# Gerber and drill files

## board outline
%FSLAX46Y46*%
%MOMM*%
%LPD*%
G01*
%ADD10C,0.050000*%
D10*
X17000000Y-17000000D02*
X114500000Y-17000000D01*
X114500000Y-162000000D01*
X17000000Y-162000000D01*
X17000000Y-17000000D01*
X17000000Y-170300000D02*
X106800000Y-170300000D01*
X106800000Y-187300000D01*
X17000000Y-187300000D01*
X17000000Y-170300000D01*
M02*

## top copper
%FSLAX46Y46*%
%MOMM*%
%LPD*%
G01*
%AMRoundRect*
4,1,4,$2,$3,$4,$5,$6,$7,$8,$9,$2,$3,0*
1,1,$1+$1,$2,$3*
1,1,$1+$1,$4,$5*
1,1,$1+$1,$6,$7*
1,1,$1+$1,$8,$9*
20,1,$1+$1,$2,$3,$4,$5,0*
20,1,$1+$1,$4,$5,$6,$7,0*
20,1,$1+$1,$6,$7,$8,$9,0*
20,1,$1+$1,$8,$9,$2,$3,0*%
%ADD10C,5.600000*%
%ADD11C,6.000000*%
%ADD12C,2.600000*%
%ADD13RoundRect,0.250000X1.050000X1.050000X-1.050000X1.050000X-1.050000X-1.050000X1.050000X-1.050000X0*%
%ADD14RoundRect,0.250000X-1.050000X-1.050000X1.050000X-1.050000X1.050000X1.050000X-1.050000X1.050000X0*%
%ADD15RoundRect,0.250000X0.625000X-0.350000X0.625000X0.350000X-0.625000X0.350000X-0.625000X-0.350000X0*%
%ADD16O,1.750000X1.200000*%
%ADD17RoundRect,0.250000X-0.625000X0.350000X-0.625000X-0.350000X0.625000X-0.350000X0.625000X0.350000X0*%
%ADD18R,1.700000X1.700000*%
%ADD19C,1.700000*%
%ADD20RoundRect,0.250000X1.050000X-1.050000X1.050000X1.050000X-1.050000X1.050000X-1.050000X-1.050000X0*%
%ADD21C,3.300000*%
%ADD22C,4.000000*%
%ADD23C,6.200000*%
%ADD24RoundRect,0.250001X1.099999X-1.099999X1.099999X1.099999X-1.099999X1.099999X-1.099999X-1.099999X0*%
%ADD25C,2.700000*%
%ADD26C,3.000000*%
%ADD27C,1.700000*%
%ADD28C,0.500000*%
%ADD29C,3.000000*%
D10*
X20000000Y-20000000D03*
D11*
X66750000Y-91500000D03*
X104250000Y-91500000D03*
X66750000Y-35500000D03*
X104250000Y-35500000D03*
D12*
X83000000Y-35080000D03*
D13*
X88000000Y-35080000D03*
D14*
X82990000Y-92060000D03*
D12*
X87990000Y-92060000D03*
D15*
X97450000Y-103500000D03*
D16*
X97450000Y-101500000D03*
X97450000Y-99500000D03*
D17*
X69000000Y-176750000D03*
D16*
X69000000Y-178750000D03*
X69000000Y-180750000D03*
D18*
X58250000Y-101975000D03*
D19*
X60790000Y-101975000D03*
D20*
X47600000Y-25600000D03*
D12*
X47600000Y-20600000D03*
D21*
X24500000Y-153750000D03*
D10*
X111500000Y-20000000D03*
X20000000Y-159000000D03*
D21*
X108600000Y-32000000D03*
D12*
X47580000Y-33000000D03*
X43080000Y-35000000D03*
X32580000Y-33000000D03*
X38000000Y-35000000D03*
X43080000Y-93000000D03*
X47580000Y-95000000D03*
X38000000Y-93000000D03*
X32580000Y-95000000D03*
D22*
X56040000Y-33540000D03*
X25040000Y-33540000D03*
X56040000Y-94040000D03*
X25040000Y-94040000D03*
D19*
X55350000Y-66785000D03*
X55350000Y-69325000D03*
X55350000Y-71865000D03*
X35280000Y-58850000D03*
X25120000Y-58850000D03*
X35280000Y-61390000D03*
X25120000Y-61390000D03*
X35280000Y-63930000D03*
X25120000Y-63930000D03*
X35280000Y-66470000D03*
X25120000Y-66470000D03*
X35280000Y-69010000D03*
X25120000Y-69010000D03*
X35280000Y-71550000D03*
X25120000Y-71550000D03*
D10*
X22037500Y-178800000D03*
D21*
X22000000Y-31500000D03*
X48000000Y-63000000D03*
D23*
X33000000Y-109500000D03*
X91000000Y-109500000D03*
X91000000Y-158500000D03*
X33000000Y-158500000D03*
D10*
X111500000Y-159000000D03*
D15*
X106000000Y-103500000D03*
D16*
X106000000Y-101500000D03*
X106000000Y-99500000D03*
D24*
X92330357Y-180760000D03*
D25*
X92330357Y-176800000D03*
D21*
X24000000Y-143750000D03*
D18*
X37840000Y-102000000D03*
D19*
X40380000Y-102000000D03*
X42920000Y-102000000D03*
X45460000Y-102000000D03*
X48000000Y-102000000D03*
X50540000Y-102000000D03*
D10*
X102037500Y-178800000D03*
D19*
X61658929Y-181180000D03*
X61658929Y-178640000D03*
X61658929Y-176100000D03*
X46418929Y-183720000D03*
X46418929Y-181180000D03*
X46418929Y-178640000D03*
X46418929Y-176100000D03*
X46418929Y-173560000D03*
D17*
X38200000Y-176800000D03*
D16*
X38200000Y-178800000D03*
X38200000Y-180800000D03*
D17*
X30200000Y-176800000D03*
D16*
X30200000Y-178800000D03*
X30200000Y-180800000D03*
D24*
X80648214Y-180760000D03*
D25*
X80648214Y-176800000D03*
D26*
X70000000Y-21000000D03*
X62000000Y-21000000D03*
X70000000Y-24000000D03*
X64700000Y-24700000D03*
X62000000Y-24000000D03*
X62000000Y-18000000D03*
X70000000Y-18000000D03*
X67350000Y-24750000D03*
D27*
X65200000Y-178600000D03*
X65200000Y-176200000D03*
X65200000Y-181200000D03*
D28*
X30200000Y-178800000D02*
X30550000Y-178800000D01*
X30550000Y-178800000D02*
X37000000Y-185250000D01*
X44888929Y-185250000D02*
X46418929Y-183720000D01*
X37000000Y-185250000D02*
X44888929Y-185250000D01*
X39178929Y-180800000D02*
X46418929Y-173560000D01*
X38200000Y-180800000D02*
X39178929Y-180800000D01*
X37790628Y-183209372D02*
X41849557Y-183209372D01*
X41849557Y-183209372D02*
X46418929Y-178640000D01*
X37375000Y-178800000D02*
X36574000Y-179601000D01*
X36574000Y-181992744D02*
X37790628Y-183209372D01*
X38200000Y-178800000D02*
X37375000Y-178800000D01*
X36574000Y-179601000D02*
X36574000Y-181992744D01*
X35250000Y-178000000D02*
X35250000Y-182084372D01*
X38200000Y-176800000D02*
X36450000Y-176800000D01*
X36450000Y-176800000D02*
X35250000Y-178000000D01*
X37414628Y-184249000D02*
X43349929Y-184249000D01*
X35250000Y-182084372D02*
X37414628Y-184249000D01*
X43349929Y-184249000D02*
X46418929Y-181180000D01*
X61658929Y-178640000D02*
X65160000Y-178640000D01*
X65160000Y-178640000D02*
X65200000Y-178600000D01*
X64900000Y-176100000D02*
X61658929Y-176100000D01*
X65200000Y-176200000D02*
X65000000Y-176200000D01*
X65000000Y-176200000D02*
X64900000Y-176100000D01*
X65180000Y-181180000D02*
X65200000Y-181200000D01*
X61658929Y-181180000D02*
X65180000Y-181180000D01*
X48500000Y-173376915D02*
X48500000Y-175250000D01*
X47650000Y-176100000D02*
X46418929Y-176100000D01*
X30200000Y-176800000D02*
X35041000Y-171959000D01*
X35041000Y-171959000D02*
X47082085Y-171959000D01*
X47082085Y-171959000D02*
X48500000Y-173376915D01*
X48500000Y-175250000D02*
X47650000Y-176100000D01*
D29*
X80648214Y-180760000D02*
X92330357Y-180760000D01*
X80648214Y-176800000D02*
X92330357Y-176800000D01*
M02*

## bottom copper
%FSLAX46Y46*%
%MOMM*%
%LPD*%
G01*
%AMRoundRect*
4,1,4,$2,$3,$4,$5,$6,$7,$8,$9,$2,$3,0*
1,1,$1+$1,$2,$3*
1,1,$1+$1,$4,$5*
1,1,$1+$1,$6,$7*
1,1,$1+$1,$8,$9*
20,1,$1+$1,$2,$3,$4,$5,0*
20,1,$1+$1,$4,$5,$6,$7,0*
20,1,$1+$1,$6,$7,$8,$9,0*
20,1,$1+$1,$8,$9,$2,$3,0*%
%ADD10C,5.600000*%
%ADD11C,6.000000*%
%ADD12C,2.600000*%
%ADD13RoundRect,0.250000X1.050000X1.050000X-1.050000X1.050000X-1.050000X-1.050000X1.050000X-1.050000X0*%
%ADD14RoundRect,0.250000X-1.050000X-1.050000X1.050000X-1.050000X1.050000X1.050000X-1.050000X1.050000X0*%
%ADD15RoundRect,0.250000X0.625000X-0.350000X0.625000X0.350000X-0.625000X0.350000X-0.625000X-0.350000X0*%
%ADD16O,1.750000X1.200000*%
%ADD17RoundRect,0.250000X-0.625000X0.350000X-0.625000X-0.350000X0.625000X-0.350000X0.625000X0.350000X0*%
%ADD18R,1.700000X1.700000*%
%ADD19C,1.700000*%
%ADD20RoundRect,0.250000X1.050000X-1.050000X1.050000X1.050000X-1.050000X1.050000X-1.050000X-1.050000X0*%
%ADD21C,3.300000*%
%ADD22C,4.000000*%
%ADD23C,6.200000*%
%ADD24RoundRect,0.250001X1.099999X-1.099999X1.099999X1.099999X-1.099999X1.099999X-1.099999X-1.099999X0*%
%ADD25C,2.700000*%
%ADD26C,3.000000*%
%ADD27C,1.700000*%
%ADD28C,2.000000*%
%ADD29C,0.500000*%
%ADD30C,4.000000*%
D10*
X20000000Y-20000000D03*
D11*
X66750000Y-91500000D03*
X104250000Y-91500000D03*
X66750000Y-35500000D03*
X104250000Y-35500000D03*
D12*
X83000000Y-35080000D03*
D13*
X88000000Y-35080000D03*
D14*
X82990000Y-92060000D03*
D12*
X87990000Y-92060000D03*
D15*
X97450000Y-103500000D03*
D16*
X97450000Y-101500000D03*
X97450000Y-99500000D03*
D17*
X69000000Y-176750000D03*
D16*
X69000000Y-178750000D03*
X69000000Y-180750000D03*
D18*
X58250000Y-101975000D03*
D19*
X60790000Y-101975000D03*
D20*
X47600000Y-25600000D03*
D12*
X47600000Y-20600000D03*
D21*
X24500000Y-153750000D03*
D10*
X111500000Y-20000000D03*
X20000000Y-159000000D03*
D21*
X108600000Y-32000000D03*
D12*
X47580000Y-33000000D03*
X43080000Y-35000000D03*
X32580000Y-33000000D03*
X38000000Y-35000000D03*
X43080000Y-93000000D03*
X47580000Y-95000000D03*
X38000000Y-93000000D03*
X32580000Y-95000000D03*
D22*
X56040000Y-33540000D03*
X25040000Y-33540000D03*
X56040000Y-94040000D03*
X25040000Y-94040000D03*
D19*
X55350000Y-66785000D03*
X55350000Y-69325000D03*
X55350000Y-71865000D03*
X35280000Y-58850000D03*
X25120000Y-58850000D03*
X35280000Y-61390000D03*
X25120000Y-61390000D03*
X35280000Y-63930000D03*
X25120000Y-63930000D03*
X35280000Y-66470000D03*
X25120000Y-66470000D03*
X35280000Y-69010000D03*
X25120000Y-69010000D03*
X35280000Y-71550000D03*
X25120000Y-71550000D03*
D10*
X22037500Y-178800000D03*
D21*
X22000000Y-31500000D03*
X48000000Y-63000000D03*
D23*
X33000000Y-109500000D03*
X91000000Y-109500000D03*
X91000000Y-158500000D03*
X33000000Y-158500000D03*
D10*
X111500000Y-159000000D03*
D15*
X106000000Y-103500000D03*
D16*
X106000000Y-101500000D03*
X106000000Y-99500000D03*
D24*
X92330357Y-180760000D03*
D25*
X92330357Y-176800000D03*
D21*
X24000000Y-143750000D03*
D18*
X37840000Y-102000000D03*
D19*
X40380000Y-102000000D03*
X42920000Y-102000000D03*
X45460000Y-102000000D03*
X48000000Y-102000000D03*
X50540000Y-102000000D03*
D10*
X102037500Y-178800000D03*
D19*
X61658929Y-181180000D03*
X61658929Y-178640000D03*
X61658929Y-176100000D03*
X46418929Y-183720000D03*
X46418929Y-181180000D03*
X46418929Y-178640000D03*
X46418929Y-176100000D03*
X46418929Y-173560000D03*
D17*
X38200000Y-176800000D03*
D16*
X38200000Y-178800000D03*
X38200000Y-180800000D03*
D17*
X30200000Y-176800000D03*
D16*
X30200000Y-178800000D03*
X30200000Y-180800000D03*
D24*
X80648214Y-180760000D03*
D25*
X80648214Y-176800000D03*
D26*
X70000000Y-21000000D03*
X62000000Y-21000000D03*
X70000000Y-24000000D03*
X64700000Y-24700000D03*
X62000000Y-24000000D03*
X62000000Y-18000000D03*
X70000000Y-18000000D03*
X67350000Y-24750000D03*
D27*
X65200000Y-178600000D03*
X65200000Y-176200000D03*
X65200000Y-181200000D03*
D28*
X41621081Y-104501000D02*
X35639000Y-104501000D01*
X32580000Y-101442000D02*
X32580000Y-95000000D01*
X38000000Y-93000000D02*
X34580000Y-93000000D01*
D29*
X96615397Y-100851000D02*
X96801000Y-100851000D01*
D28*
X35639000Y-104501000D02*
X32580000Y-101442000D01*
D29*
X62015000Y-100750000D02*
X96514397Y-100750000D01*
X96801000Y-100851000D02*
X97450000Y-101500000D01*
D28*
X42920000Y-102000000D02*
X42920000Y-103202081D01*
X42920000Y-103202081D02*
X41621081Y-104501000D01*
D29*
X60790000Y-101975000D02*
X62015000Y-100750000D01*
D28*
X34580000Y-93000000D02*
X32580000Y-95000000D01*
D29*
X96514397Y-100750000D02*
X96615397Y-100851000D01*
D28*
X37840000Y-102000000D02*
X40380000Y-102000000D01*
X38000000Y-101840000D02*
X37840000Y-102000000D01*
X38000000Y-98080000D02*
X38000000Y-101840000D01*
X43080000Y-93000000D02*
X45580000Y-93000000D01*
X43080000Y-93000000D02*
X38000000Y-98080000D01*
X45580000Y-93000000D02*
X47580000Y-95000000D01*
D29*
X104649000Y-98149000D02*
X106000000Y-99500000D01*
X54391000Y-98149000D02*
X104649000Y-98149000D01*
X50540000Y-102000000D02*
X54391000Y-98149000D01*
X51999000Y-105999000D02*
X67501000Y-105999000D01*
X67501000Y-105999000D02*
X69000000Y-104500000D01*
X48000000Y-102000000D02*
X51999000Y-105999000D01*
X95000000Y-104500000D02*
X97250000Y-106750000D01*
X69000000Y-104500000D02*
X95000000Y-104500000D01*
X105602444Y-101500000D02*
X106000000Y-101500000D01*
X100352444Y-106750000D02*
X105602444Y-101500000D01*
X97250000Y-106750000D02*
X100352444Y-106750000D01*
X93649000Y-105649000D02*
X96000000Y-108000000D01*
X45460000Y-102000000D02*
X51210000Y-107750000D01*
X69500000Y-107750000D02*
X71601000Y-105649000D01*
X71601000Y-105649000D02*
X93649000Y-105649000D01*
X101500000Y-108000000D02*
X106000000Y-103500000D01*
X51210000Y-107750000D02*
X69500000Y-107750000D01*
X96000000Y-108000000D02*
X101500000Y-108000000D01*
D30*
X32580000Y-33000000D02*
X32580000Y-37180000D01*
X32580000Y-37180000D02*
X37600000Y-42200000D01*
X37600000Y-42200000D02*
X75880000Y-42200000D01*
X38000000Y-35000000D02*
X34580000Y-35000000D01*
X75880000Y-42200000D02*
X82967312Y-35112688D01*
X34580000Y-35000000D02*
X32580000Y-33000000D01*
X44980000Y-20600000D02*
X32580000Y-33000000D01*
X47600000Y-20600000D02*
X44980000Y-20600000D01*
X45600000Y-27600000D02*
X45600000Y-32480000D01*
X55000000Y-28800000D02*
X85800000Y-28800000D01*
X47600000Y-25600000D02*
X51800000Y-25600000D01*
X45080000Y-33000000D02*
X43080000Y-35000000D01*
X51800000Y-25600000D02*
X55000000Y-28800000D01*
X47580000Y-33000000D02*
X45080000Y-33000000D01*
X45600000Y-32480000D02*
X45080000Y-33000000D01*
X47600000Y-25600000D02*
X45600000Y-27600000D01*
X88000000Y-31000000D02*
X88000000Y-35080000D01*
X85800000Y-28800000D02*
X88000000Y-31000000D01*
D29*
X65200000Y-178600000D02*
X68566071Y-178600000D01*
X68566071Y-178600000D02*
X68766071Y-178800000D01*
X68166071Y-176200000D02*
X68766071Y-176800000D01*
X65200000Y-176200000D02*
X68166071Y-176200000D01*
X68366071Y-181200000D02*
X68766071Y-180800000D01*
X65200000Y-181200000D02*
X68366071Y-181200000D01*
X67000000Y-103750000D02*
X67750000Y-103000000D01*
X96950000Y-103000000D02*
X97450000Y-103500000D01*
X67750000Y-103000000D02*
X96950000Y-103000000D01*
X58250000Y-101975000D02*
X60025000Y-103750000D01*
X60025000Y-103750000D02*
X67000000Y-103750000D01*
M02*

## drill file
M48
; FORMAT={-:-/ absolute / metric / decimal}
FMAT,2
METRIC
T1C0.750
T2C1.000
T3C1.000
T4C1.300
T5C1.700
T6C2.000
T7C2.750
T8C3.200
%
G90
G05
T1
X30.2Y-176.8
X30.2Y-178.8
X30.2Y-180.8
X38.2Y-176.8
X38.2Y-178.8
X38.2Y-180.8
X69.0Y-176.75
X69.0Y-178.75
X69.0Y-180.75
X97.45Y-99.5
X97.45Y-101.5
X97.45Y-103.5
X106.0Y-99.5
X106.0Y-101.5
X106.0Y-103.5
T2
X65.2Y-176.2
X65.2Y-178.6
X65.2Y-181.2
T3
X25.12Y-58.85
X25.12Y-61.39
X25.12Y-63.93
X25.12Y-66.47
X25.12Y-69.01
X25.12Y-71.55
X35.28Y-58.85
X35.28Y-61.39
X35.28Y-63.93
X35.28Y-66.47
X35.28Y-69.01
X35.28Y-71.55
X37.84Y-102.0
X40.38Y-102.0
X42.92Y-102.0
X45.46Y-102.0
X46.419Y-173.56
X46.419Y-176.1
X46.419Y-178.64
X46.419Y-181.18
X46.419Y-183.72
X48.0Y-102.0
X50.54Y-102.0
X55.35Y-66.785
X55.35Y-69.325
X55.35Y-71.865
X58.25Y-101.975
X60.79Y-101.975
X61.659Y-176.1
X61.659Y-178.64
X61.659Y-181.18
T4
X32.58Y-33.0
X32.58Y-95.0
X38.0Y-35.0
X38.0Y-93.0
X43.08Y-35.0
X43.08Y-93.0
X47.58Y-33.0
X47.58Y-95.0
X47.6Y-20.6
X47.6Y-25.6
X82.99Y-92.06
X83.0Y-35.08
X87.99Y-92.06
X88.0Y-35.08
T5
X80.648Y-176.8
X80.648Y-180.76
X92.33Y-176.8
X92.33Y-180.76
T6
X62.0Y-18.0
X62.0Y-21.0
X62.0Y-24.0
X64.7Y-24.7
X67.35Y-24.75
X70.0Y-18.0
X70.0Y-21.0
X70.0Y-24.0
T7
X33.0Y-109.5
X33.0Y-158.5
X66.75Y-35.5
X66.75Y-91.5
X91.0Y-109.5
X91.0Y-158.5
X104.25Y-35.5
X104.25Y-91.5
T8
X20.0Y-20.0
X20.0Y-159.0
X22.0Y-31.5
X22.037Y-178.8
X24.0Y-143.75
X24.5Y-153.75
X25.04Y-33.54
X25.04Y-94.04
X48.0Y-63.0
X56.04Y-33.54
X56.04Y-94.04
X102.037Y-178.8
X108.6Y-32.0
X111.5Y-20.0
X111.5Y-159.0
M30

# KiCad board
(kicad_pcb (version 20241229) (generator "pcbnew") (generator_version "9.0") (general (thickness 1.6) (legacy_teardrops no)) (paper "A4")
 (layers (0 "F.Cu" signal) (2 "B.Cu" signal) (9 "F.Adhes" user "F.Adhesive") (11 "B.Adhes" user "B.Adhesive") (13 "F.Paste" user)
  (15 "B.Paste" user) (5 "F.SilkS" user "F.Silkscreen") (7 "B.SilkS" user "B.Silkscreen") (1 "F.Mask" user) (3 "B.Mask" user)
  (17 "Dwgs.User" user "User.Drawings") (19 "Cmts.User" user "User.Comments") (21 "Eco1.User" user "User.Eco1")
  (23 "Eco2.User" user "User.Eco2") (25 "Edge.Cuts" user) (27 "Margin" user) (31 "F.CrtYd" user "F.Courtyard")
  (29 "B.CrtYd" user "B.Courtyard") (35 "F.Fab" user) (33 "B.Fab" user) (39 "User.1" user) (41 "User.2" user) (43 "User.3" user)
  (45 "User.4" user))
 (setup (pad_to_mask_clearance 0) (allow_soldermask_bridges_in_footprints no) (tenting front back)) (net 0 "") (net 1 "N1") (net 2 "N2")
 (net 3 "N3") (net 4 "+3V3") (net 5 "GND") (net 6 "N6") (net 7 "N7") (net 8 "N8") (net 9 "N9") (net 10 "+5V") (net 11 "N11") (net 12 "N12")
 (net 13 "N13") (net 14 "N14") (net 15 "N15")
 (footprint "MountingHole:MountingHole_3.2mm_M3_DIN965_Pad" (layer "F.Cu") (at 20 20)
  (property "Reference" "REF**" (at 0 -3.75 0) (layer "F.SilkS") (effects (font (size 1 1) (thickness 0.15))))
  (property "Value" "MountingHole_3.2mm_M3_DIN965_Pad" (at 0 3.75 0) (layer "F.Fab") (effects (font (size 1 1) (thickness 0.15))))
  (pad "1" thru_hole circle (at 0 0) (size 5.6 5.6) (drill 3.2) (layers "*.Cu" "*.Mask") (remove_unused_layers no) (zone_connect 2)))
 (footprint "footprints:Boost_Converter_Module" (layer "F.Cu") (at 85.5 63.5 90)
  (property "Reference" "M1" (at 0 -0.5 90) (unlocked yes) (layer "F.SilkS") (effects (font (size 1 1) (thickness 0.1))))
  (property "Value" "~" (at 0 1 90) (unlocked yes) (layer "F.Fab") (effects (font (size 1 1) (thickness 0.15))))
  (pad "" thru_hole circle (at -28 -18.75 90) (size 6 6) (drill 2.75) (layers "*.Cu" "*.Mask") (remove_unused_layers no))
  (pad "" thru_hole circle (at -28 18.75 90) (size 6 6) (drill 2.75) (layers "*.Cu" "*.Mask") (remove_unused_layers no))
  (pad "" thru_hole circle (at 28 -18.75 90) (size 6 6) (drill 2.75) (layers "*.Cu" "*.Mask") (remove_unused_layers no))
  (pad "" thru_hole circle (at 28 18.75 90) (size 6 6) (drill 2.75) (layers "*.Cu" "*.Mask") (remove_unused_layers no))
  (pad "1" thru_hole circle (at 28.42 -2.5 180) (size 2.6 2.6) (drill 1.3) (layers "*.Cu" "*.Mask") (remove_unused_layers no) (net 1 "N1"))
  (pad "2" thru_hole roundrect (at 28.42 2.5 180) (size 2.6 2.6) (drill 1.3) (layers "*.Cu" "*.Mask") (remove_unused_layers no)
   (roundrect_rratio 0.096154) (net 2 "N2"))
  (pad "3" thru_hole roundrect (at -28.56 -2.51) (size 2.6 2.6) (drill 1.3) (layers "*.Cu" "*.Mask") (remove_unused_layers no)
   (roundrect_rratio 0.096154) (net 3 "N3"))
  (pad "4" thru_hole circle (at -28.56 2.49) (size 2.6 2.6) (drill 1.3) (layers "*.Cu" "*.Mask") (remove_unused_layers no)))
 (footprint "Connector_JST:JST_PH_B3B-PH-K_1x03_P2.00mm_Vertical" (layer "F.Cu") (at 97.45 103.5 90)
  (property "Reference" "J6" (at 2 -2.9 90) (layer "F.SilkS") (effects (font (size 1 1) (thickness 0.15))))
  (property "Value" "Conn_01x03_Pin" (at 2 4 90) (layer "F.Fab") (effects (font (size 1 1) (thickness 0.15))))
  (pad "1" thru_hole roundrect (at 0 0 90) (size 1.2 1.75) (drill 0.75) (layers "*.Cu" "*.Mask") (remove_unused_layers no)
   (roundrect_rratio 0.208333) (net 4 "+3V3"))
  (pad "2" thru_hole oval (at 2 0 90) (size 1.2 1.75) (drill 0.75) (layers "*.Cu" "*.Mask") (remove_unused_layers no) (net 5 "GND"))
  (pad "3" thru_hole oval (at 4 0 90) (size 1.2 1.75) (drill 0.75) (layers "*.Cu" "*.Mask") (remove_unused_layers no) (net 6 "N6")))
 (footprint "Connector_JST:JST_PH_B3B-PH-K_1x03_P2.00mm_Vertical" (layer "F.Cu") (at 69 176.75 -90)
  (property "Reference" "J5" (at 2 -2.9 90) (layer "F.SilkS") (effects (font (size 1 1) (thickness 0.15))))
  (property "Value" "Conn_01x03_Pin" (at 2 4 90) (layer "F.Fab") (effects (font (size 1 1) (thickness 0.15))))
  (pad "1" thru_hole roundrect (at 0 0 270) (size 1.2 1.75) (drill 0.75) (layers "*.Cu" "*.Mask") (remove_unused_layers no)
   (roundrect_rratio 0.208333) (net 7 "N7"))
  (pad "2" thru_hole oval (at 2 0 270) (size 1.2 1.75) (drill 0.75) (layers "*.Cu" "*.Mask") (remove_unused_layers no) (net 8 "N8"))
  (pad "3" thru_hole oval (at 4 0 270) (size 1.2 1.75) (drill 0.75) (layers "*.Cu" "*.Mask") (remove_unused_layers no) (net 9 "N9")))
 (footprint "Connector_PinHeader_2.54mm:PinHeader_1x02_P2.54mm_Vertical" (layer "F.Cu") (at 58.25 101.975 90)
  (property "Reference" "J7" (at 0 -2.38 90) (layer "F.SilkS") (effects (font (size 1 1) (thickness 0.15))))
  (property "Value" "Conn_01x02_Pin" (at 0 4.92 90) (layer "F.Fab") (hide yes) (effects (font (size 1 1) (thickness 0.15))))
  (pad "1" thru_hole rect (at 0 0 90) (size 1.7 1.7) (drill 1) (layers "*.Cu" "*.Mask") (remove_unused_layers no) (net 4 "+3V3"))
  (pad "2" thru_hole circle (at 0 2.54 90) (size 1.7 1.7) (drill 1) (layers "*.Cu" "*.Mask") (remove_unused_layers no) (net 5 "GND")))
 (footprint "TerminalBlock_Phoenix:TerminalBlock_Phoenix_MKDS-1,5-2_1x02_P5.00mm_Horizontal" (layer "F.Cu") (at 47.6 25.6 90)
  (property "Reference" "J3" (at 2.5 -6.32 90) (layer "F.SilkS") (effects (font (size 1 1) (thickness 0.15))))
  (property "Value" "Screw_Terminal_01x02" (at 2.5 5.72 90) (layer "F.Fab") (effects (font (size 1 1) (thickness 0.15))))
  (pad "1" thru_hole roundrect (at 0 0 90) (size 2.6 2.6) (drill 1.3) (layers "*.Cu" "*.Mask") (remove_unused_layers no)
   (roundrect_rratio 0.096154) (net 2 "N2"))
  (pad "2" thru_hole circle (at 5 0 90) (size 2.6 2.6) (drill 1.3) (layers "*.Cu" "*.Mask") (remove_unused_layers no) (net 1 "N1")))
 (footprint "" (layer "F.Cu") (at 24.5 153.75)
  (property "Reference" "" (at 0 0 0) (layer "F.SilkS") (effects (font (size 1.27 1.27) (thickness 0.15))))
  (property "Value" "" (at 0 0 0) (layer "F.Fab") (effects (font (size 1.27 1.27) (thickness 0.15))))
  (pad "1" thru_hole circle (at 0 0) (size 3.3 3.3) (drill 3.2) (layers "*.Cu" "*.Mask") (remove_unused_layers no) (zone_connect 2)))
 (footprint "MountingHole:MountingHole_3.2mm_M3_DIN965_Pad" (layer "F.Cu") (at 111.5 20)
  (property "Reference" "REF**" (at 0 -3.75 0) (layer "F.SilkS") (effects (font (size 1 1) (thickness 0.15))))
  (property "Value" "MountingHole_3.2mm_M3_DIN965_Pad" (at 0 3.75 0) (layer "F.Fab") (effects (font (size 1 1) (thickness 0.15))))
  (pad "1" thru_hole circle (at 0 0) (size 5.6 5.6) (drill 3.2) (layers "*.Cu" "*.Mask") (remove_unused_layers no) (zone_connect 2)))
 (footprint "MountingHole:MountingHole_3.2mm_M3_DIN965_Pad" (layer "F.Cu") (at 20 159)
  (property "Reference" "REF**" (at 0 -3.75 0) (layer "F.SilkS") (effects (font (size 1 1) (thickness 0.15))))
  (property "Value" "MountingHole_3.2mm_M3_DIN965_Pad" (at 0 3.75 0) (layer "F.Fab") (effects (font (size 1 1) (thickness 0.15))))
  (pad "1" thru_hole circle (at 0 0) (size 5.6 5.6) (drill 3.2) (layers "*.Cu" "*.Mask") (remove_unused_layers no) (zone_connect 2)))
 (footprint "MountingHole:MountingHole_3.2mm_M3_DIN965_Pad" (layer "F.Cu") (at 108.6 32)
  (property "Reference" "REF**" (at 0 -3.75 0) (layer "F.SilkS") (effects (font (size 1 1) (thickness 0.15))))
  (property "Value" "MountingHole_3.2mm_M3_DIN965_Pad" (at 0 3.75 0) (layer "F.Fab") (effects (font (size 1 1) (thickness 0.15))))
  (pad "1" thru_hole circle (at 0 0) (size 3.3 3.3) (drill 3.2) (layers "*.Cu" "*.Mask") (remove_unused_layers no) (zone_connect 2)))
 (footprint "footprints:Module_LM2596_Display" (layer "F.Cu") (at 58.58 64 -90)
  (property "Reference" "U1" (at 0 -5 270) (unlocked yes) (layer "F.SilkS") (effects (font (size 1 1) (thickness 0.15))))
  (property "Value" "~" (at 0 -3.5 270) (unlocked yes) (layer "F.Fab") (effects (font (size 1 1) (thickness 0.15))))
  (pad "1" thru_hole circle (at -31 11 270) (size 2.6 2.6) (drill 1.3) (layers "*.Cu" "*.Mask") (remove_unused_layers no) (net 2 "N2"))
  (pad "1" thru_hole circle (at -29 15.5 270) (size 2.6 2.6) (drill 1.3) (layers "*.Cu" "*.Mask") (remove_unused_layers no) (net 2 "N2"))
  (pad "2" thru_hole circle (at -31 26 270) (size 2.6 2.6) (drill 1.3) (layers "*.Cu" "*.Mask") (remove_unused_layers no) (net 1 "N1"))
  (pad "2" thru_hole circle (at -29 20.58 270) (size 2.6 2.6) (drill 1.3) (layers "*.Cu" "*.Mask") (remove_unused_layers no) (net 1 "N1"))
  (pad "3" thru_hole circle (at 29 15.5 270) (size 2.6 2.6) (drill 1.3) (layers "*.Cu" "*.Mask") (remove_unused_layers no) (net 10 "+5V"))
  (pad "3" thru_hole circle (at 31 11 270) (size 2.6 2.6) (drill 1.3) (layers "*.Cu" "*.Mask") (remove_unused_layers no) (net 10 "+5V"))
  (pad "4" thru_hole circle (at 29 20.58 270) (size 2.6 2.6) (drill 1.3) (layers "*.Cu" "*.Mask") (remove_unused_layers no) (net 5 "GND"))
  (pad "4" thru_hole circle (at 31 26 270) (size 2.6 2.6) (drill 1.3) (layers "*.Cu" "*.Mask") (remove_unused_layers no) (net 5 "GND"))
  (pad "5" thru_hole circle (at -30.46 2.54 270) (size 4 4) (drill 3.2) (layers "*.Cu" "*.Mask") (remove_unused_layers no))
  (pad "5" thru_hole circle (at -30.46 33.54 270) (size 4 4) (drill 3.2) (layers "*.Cu" "*.Mask") (remove_unused_layers no))
  (pad "5" thru_hole circle (at 30.04 2.54 270) (size 4 4) (drill 3.2) (layers "*.Cu" "*.Mask") (remove_unused_layers no))
  (pad "5" thru_hole circle (at 30.04 33.54 270) (size 4 4) (drill 3.2) (layers "*.Cu" "*.Mask") (remove_unused_layers no))
  (pad "6" thru_hole circle (at 2.785 3.23 90) (size 1.7 1.7) (drill 1) (layers "*.Cu" "*.Mask") (remove_unused_layers no))
  (pad "7" thru_hole circle (at 5.325 3.23 90) (size 1.7 1.7) (drill 1) (layers "*.Cu" "*.Mask") (remove_unused_layers no))
  (pad "8" thru_hole circle (at 7.865 3.23 90) (size 1.7 1.7) (drill 1) (layers "*.Cu" "*.Mask") (remove_unused_layers no))
  (pad "9" thru_hole circle (at -5.15 23.3 270) (size 1.7 1.7) (drill 1) (layers "*.Cu" "*.Mask") (remove_unused_layers no))
  (pad "9" thru_hole circle (at -5.15 33.46 270) (size 1.7 1.7) (drill 1) (layers "*.Cu" "*.Mask") (remove_unused_layers no))
  (pad "9" thru_hole circle (at -2.61 23.3 270) (size 1.7 1.7) (drill 1) (layers "*.Cu" "*.Mask") (remove_unused_layers no))
  (pad "9" thru_hole circle (at -2.61 33.46 270) (size 1.7 1.7) (drill 1) (layers "*.Cu" "*.Mask") (remove_unused_layers no))
  (pad "9" thru_hole circle (at -0.07 23.3 270) (size 1.7 1.7) (drill 1) (layers "*.Cu" "*.Mask") (remove_unused_layers no))
  (pad "9" thru_hole circle (at -0.07 33.46 270) (size 1.7 1.7) (drill 1) (layers "*.Cu" "*.Mask") (remove_unused_layers no))
  (pad "9" thru_hole circle (at 2.47 23.3 270) (size 1.7 1.7) (drill 1) (layers "*.Cu" "*.Mask" "Eco1.User") (remove_unused_layers no))
  (pad "9" thru_hole circle (at 2.47 33.46 270) (size 1.7 1.7) (drill 1) (layers "*.Cu" "*.Mask") (remove_unused_layers no))
  (pad "9" thru_hole circle (at 5.01 23.3 270) (size 1.7 1.7) (drill 1) (layers "*.Cu" "*.Mask") (remove_unused_layers no))
  (pad "9" thru_hole circle (at 5.01 33.46 270) (size 1.7 1.7) (drill 1) (layers "*.Cu" "*.Mask") (remove_unused_layers no))
  (pad "9" thru_hole circle (at 7.55 23.3 270) (size 1.7 1.7) (drill 1) (layers "*.Cu" "*.Mask") (remove_unused_layers no))
  (pad "9" thru_hole circle (at 7.55 33.46 270) (size 1.7 1.7) (drill 1) (layers "*.Cu" "*.Mask") (remove_unused_layers no)))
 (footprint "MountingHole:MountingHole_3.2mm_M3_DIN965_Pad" (layer "F.Cu") (at 22.0375 178.8)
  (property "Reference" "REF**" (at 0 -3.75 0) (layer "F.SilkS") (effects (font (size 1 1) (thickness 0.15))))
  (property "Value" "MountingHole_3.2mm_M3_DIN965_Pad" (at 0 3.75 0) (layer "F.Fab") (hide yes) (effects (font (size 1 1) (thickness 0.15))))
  (pad "1" thru_hole circle (at 0 0) (size 5.6 5.6) (drill 3.2) (layers "*.Cu" "*.Mask") (remove_unused_layers no) (zone_connect 2)))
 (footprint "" (layer "F.Cu") (at 22 31.5)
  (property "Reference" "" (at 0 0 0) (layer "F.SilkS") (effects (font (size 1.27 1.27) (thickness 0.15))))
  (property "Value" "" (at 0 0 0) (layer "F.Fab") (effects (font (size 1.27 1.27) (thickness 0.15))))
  (pad "1" thru_hole circle (at 0 0) (size 3.3 3.3) (drill 3.2) (layers "*.Cu" "*.Mask") (remove_unused_layers no) (zone_connect 2)))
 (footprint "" (layer "F.Cu") (at 48 63)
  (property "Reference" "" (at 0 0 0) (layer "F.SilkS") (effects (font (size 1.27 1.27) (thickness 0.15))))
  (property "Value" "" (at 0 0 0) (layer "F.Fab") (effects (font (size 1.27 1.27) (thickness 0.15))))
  (pad "1" thru_hole circle (at 0 0) (size 3.3 3.3) (drill 3.2) (layers "*.Cu" "*.Mask") (remove_unused_layers no) (zone_connect 2)))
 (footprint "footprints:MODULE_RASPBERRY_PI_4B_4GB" (layer "F.Cu") (at 72 134)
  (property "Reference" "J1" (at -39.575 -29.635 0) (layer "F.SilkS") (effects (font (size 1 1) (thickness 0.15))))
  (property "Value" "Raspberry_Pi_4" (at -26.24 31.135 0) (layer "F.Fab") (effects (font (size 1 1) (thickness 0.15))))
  (pad "S1" thru_hole circle (at -39 -24.5) (size 6.2 6.2) (drill 2.75) (layers "*.Cu" "*.Mask") (remove_unused_layers no)
   (solder_mask_margin 0.102))
  (pad "S2" thru_hole circle (at 19 -24.5) (size 6.2 6.2) (drill 2.75) (layers "*.Cu" "*.Mask") (remove_unused_layers no)
   (solder_mask_margin 0.102))
  (pad "S3" thru_hole circle (at 19 24.5) (size 6.2 6.2) (drill 2.75) (layers "*.Cu" "*.Mask") (remove_unused_layers no)
   (solder_mask_margin 0.102))
  (pad "S4" thru_hole circle (at -39 24.5) (size 6.2 6.2) (drill 2.75) (layers "*.Cu" "*.Mask") (remove_unused_layers no)
   (solder_mask_margin 0.102)))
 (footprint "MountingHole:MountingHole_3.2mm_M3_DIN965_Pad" (layer "F.Cu") (at 111.5 159)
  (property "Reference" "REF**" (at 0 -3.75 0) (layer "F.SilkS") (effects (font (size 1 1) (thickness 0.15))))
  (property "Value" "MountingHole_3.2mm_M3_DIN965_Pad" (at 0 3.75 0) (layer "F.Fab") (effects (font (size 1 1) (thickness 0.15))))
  (pad "1" thru_hole circle (at 0 0) (size 5.6 5.6) (drill 3.2) (layers "*.Cu" "*.Mask") (remove_unused_layers no) (zone_connect 2)))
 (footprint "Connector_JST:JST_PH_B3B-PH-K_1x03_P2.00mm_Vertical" (layer "F.Cu") (at 106 103.5 90)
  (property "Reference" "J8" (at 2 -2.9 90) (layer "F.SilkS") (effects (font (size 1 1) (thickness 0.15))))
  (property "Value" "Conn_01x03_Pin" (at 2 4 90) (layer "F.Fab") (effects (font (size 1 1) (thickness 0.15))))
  (pad "1" thru_hole roundrect (at 0 0 90) (size 1.2 1.75) (drill 0.75) (layers "*.Cu" "*.Mask") (remove_unused_layers no)
   (roundrect_rratio 0.208333) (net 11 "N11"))
  (pad "2" thru_hole oval (at 2 0 90) (size 1.2 1.75) (drill 0.75) (layers "*.Cu" "*.Mask") (remove_unused_layers no) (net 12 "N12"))
  (pad "3" thru_hole oval (at 4 0 90) (size 1.2 1.75) (drill 0.75) (layers "*.Cu" "*.Mask") (remove_unused_layers no) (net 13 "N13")))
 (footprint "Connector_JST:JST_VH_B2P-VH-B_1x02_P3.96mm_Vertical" (layer "F.Cu") (at 92.330357 180.76 90)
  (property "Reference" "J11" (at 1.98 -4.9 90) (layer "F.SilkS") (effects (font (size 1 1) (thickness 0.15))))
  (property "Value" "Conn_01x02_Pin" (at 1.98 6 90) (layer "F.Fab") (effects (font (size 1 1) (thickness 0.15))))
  (pad "1" thru_hole roundrect (at 0 0 90) (size 2.7 2.7) (drill 1.7) (layers "*.Cu" "*.Mask") (remove_unused_layers no)
   (roundrect_rratio 0.092593) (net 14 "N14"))
  (pad "2" thru_hole circle (at 3.96 0 90) (size 2.7 2.7) (drill 1.7) (layers "*.Cu" "*.Mask") (remove_unused_layers no) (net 3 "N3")))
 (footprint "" (layer "F.Cu") (at 24 143.75)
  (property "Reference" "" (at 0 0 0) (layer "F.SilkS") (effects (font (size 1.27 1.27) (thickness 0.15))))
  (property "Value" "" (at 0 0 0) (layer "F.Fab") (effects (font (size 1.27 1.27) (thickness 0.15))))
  (pad "1" thru_hole circle (at 0 0) (size 3.3 3.3) (drill 3.2) (layers "*.Cu" "*.Mask") (remove_unused_layers no) (zone_connect 2)))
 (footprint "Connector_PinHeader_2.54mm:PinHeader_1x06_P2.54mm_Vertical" (layer "F.Cu") (at 37.84 102 90)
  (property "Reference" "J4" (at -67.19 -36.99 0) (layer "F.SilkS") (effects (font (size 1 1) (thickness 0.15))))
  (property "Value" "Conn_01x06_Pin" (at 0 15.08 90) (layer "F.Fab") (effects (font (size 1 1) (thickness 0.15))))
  (pad "1" thru_hole rect (at 0 0 90) (size 1.7 1.7) (drill 1) (layers "*.Cu" "*.Mask") (remove_unused_layers no) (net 10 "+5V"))
  (pad "2" thru_hole circle (at 0 2.54 90) (size 1.7 1.7) (drill 1) (layers "*.Cu" "*.Mask") (remove_unused_layers no) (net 10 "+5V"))
  (pad "3" thru_hole circle (at 0 5.08 90) (size 1.7 1.7) (drill 1) (layers "*.Cu" "*.Mask") (remove_unused_layers no) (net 5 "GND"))
  (pad "4" thru_hole circle (at 0 7.62 90) (size 1.7 1.7) (drill 1) (layers "*.Cu" "*.Mask") (remove_unused_layers no) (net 11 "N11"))
  (pad "5" thru_hole circle (at 0 10.16 90) (size 1.7 1.7) (drill 1) (layers "*.Cu" "*.Mask") (remove_unused_layers no) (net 12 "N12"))
  (pad "6" thru_hole circle (at 0 12.7 90) (size 1.7 1.7) (drill 1) (layers "*.Cu" "*.Mask") (remove_unused_layers no) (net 13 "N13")))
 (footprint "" (layer "F.Cu") (at 102.0375 178.8)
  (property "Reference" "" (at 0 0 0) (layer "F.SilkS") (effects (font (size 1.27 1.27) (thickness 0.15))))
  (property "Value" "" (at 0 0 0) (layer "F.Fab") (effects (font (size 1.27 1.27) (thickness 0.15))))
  (pad "1" thru_hole circle (at 0 0) (size 5.6 5.6) (drill 3.2) (layers "*.Cu" "*.Mask") (remove_unused_layers no) (zone_connect 2)))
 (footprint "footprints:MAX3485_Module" (layer "B.Cu") (at 57.658929 174.14 90)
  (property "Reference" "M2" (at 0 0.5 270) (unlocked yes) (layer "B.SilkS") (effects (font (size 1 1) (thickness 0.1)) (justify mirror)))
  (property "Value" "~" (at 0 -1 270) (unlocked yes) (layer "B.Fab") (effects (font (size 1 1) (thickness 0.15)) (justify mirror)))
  (pad "1" thru_hole circle (at -7.04 4 90) (size 1.7 1.7) (drill 1) (layers "*.Cu" "*.Mask") (remove_unused_layers no) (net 7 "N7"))
  (pad "2" thru_hole circle (at -4.5 4 90) (size 1.7 1.7) (drill 1) (layers "*.Cu" "*.Mask") (remove_unused_layers no) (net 8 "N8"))
  (pad "3" thru_hole circle (at -1.96 4 90) (size 1.7 1.7) (drill 1) (layers "*.Cu" "*.Mask") (remove_unused_layers no) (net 9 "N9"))
  (pad "4" thru_hole circle (at -9.58 -11.24 90) (size 1.7 1.7) (drill 1) (layers "*.Cu" "*.Mask") (remove_unused_layers no) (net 5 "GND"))
  (pad "5" thru_hole circle (at -7.04 -11.24 90) (size 1.7 1.7) (drill 1) (layers "*.Cu" "*.Mask") (remove_unused_layers no) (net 11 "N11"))
  (pad "6" thru_hole circle (at -4.5 -11.24 90) (size 1.7 1.7) (drill 1) (layers "*.Cu" "*.Mask") (remove_unused_layers no) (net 12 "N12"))
  (pad "7" thru_hole circle (at -1.96 -11.24 90) (size 1.7 1.7) (drill 1) (layers "*.Cu" "*.Mask") (remove_unused_layers no) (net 4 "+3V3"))
  (pad "8" thru_hole circle (at 0.58 -11.24 90) (size 1.7 1.7) (drill 1) (layers "*.Cu" "*.Mask") (remove_unused_layers no) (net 13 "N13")))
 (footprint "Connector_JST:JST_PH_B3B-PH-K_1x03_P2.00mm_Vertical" (layer "B.Cu") (at 38.2 176.8 -90)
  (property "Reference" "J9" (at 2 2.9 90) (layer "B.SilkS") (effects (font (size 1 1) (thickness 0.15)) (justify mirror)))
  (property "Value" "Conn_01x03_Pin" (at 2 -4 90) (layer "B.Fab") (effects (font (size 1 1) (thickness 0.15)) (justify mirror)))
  (pad "1" thru_hole roundrect (at 0 0 270) (size 1.2 1.75) (drill 0.75) (layers "*.Cu" "*.Mask") (remove_unused_layers no)
   (roundrect_rratio 0.208333) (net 11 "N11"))
  (pad "2" thru_hole oval (at 2 0 270) (size 1.2 1.75) (drill 0.75) (layers "*.Cu" "*.Mask") (remove_unused_layers no) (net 12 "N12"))
  (pad "3" thru_hole oval (at 4 0 270) (size 1.2 1.75) (drill 0.75) (layers "*.Cu" "*.Mask") (remove_unused_layers no) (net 13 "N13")))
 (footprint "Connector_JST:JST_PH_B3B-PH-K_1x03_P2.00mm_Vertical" (layer "B.Cu") (at 30.2 176.8 -90)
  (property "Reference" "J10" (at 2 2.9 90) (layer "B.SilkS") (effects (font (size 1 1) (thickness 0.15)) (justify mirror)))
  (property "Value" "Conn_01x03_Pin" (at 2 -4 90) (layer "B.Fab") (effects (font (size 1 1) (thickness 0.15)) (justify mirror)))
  (pad "1" thru_hole roundrect (at 0 0 270) (size 1.2 1.75) (drill 0.75) (layers "*.Cu" "*.Mask") (remove_unused_layers no)
   (roundrect_rratio 0.208333) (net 4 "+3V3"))
  (pad "2" thru_hole oval (at 2 0 270) (size 1.2 1.75) (drill 0.75) (layers "*.Cu" "*.Mask") (remove_unused_layers no) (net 5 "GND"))
  (pad "3" thru_hole oval (at 4 0 270) (size 1.2 1.75) (drill 0.75) (layers "*.Cu" "*.Mask") (remove_unused_layers no) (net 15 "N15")))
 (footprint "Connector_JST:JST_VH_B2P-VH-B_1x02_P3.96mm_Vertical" (layer "B.Cu") (at 80.648214 180.76 90)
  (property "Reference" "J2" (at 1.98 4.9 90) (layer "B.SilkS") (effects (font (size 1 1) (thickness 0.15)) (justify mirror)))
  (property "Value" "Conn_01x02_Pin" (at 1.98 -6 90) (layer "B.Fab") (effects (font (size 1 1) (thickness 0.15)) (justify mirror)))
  (pad "1" thru_hole roundrect (at 0 0 90) (size 2.7 2.7) (drill 1.7) (layers "*.Cu" "*.Mask") (remove_unused_layers no)
   (roundrect_rratio 0.092593) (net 14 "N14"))
  (pad "2" thru_hole circle (at 3.96 0 90) (size 2.7 2.7) (drill 1.7) (layers "*.Cu" "*.Mask") (remove_unused_layers no) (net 3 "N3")))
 (gr_rect (start 17 17) (end 114.5 162) (stroke (width 0.05) (type solid)) (fill no) (layer "Edge.Cuts"))
 (gr_rect (start 17 170.3) (end 106.8 187.3) (stroke (width 0.05) (type default)) (fill no) (layer "Edge.Cuts"))
 (via (at 70 21) (size 3) (drill 2) (layers "F.Cu" "B.Cu") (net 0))
 (via (at 62 21) (size 3) (drill 2) (layers "F.Cu" "B.Cu") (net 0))
 (via (at 70 24) (size 3) (drill 2) (layers "F.Cu" "B.Cu") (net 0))
 (via (at 64.7 24.7) (size 3) (drill 2) (layers "F.Cu" "B.Cu") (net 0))
 (via (at 62 24) (size 3) (drill 2) (layers "F.Cu" "B.Cu") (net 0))
 (via (at 62 18) (size 3) (drill 2) (layers "F.Cu" "B.Cu") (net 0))
 (via (at 70 18) (size 3) (drill 2) (layers "F.Cu" "B.Cu") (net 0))
 (via (at 67.35 24.75) (size 3) (drill 2) (layers "F.Cu" "B.Cu") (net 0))
 (segment (start 30.2 178.8) (end 30.55 178.8) (width 0.5) (layer "F.Cu") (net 5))
 (segment (start 30.55 178.8) (end 37 185.25) (width 0.5) (layer "F.Cu") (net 5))
 (segment (start 44.888929 185.25) (end 46.418929 183.72) (width 0.5) (layer "F.Cu") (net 5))
 (segment (start 37 185.25) (end 44.888929 185.25) (width 0.5) (layer "F.Cu") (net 5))
 (segment (start 41.621081 104.501) (end 35.639 104.501) (width 2) (layer "B.Cu") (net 5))
 (segment (start 32.58 101.442) (end 32.58 95) (width 2) (layer "B.Cu") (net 5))
 (segment (start 38 93) (end 34.58 93) (width 2) (layer "B.Cu") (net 5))
 (segment (start 96.615397 100.851) (end 96.801 100.851) (width 0.5) (layer "B.Cu") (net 5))
 (segment (start 35.639 104.501) (end 32.58 101.442) (width 2) (layer "B.Cu") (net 5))
 (segment (start 62.015 100.75) (end 96.514397 100.75) (width 0.5) (layer "B.Cu") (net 5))
 (segment (start 96.801 100.851) (end 97.45 101.5) (width 0.5) (layer "B.Cu") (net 5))
 (segment (start 42.92 102) (end 42.92 103.202081) (width 2) (layer "B.Cu") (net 5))
 (segment (start 42.92 103.202081) (end 41.621081 104.501) (width 2) (layer "B.Cu") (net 5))
 (segment (start 60.79 101.975) (end 62.015 100.75) (width 0.5) (layer "B.Cu") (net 5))
 (segment (start 34.58 93) (end 32.58 95) (width 2) (layer "B.Cu") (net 5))
 (segment (start 96.514397 100.75) (end 96.615397 100.851) (width 0.5) (layer "B.Cu") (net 5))
 (segment (start 37.84 102) (end 40.38 102) (width 2) (layer "B.Cu") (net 10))
 (segment (start 38 101.84) (end 37.84 102) (width 2) (layer "B.Cu") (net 10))
 (segment (start 38 98.08) (end 38 101.84) (width 2) (layer "B.Cu") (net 10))
 (segment (start 43.08 93) (end 45.58 93) (width 2) (layer "B.Cu") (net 10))
 (segment (start 43.08 93) (end 38 98.08) (width 2) (layer "B.Cu") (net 10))
 (segment (start 45.58 93) (end 47.58 95) (width 2) (layer "B.Cu") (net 10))
 (segment (start 39.178929 180.8) (end 46.418929 173.56) (width 0.5) (layer "F.Cu") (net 13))
 (segment (start 38.2 180.8) (end 39.178929 180.8) (width 0.5) (layer "F.Cu") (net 13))
 (segment (start 104.649 98.149) (end 106 99.5) (width 0.5) (layer "B.Cu") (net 13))
 (segment (start 54.391 98.149) (end 104.649 98.149) (width 0.5) (layer "B.Cu") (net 13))
 (segment (start 50.54 102) (end 54.391 98.149) (width 0.5) (layer "B.Cu") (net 13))
 (segment (start 37.790628 183.209372) (end 41.849557 183.209372) (width 0.5) (layer "F.Cu") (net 12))
 (segment (start 41.849557 183.209372) (end 46.418929 178.64) (width 0.5) (layer "F.Cu") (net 12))
 (segment (start 37.375 178.8) (end 36.574 179.601) (width 0.5) (layer "F.Cu") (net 12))
 (segment (start 36.574 181.992744) (end 37.790628 183.209372) (width 0.5) (layer "F.Cu") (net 12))
 (segment (start 38.2 178.8) (end 37.375 178.8) (width 0.5) (layer "F.Cu") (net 12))
 (segment (start 36.574 179.601) (end 36.574 181.992744) (width 0.5) (layer "F.Cu") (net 12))
 (segment (start 51.999 105.999) (end 67.501 105.999) (width 0.5) (layer "B.Cu") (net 12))
 (segment (start 67.501 105.999) (end 69 104.5) (width 0.5) (layer "B.Cu") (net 12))
 (segment (start 48 102) (end 51.999 105.999) (width 0.5) (layer "B.Cu") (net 12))
 (segment (start 95 104.5) (end 97.25 106.75) (width 0.5) (layer "B.Cu") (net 12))
 (segment (start 69 104.5) (end 95 104.5) (width 0.5) (layer "B.Cu") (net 12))
 (segment (start 105.602444 101.5) (end 106 101.5) (width 0.5) (layer "B.Cu") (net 12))
 (segment (start 100.352444 106.75) (end 105.602444 101.5) (width 0.5) (layer "B.Cu") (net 12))
 (segment (start 97.25 106.75) (end 100.352444 106.75) (width 0.5) (layer "B.Cu") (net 12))
 (segment (start 35.25 178) (end 35.25 182.084372) (width 0.5) (layer "F.Cu") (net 11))
 (segment (start 38.2 176.8) (end 36.45 176.8) (width 0.5) (layer "F.Cu") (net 11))
 (segment (start 36.45 176.8) (end 35.25 178) (width 0.5) (layer "F.Cu") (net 11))
 (segment (start 37.414628 184.249) (end 43.349929 184.249) (width 0.5) (layer "F.Cu") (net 11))
 (segment (start 35.25 182.084372) (end 37.414628 184.249) (width 0.5) (layer "F.Cu") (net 11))
 (segment (start 43.349929 184.249) (end 46.418929 181.18) (width 0.5) (layer "F.Cu") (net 11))
 (segment (start 93.649 105.649) (end 96 108) (width 0.5) (layer "B.Cu") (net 11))
 (segment (start 45.46 102) (end 51.21 107.75) (width 0.5) (layer "B.Cu") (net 11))
 (segment (start 69.5 107.75) (end 71.601 105.649) (width 0.5) (layer "B.Cu") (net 11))
 (segment (start 71.601 105.649) (end 93.649 105.649) (width 0.5) (layer "B.Cu") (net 11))
 (segment (start 101.5 108) (end 106 103.5) (width 0.5) (layer "B.Cu") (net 11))
 (segment (start 51.21 107.75) (end 69.5 107.75) (width 0.5) (layer "B.Cu") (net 11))
 (segment (start 96 108) (end 101.5 108) (width 0.5) (layer "B.Cu") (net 11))
 (segment (start 32.58 33) (end 32.58 37.18) (width 4) (layer "B.Cu") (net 1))
 (segment (start 32.58 37.18) (end 37.6 42.2) (width 4) (layer "B.Cu") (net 1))
 (segment (start 37.6 42.2) (end 75.88 42.2) (width 4) (layer "B.Cu") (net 1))
 (segment (start 38 35) (end 34.58 35) (width 4) (layer "B.Cu") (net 1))
 (segment (start 75.88 42.2) (end 82.967312 35.112688) (width 4) (layer "B.Cu") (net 1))
 (segment (start 34.58 35) (end 32.58 33) (width 4) (layer "B.Cu") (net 1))
 (segment (start 44.98 20.6) (end 32.58 33) (width 4) (layer "B.Cu") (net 1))
 (segment (start 47.6 20.6) (end 44.98 20.6) (width 4) (layer "B.Cu") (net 1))
 (segment (start 45.6 27.6) (end 45.6 32.48) (width 4) (layer "B.Cu") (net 2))
 (segment (start 55 28.8) (end 85.8 28.8) (width 4) (layer "B.Cu") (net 2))
 (segment (start 47.6 25.6) (end 51.8 25.6) (width 4) (layer "B.Cu") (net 2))
 (segment (start 45.08 33) (end 43.08 35) (width 4) (layer "B.Cu") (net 2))
 (segment (start 51.8 25.6) (end 55 28.8) (width 4) (layer "B.Cu") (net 2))
 (segment (start 47.58 33) (end 45.08 33) (width 4) (layer "B.Cu") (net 2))
 (segment (start 45.6 32.48) (end 45.08 33) (width 4) (layer "B.Cu") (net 2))
 (segment (start 47.6 25.6) (end 45.6 27.6) (width 4) (layer "B.Cu") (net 2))
 (segment (start 88 31) (end 88 35.08) (width 4) (layer "B.Cu") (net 2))
 (segment (start 85.8 28.8) (end 88 31) (width 4) (layer "B.Cu") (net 2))
 (segment (start 61.658929 178.64) (end 65.16 178.64) (width 0.5) (layer "F.Cu") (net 8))
 (segment (start 65.16 178.64) (end 65.2 178.6) (width 0.5) (layer "F.Cu") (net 8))
 (via (at 65.2 178.6) (size 1.7) (drill 1) (layers "F.Cu" "B.Cu") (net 8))
 (segment (start 65.2 178.6) (end 68.566071 178.6) (width 0.5) (layer "B.Cu") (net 8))
 (segment (start 68.566071 178.6) (end 68.766071 178.8) (width 0.5) (layer "B.Cu") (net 8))
 (segment (start 64.9 176.1) (end 61.658929 176.1) (width 0.5) (layer "F.Cu") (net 9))
 (segment (start 65.2 176.2) (end 65 176.2) (width 0.5) (layer "F.Cu") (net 9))
 (segment (start 65 176.2) (end 64.9 176.1) (width 0.5) (layer "F.Cu") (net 9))
 (via (at 65.2 176.2) (size 1.7) (drill 1) (layers "F.Cu" "B.Cu") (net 9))
 (segment (start 68.166071 176.2) (end 68.766071 176.8) (width 0.5) (layer "B.Cu") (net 9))
 (segment (start 65.2 176.2) (end 68.166071 176.2) (width 0.5) (layer "B.Cu") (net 9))
 (segment (start 65.18 181.18) (end 65.2 181.2) (width 0.5) (layer "F.Cu") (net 7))
 (segment (start 61.658929 181.18) (end 65.18 181.18) (width 0.5) (layer "F.Cu") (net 7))
 (via (at 65.2 181.2) (size 1.7) (drill 1) (layers "F.Cu" "B.Cu") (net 7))
 (segment (start 68.366071 181.2) (end 68.766071 180.8) (width 0.5) (layer "B.Cu") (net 7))
 (segment (start 65.2 181.2) (end 68.366071 181.2) (width 0.5) (layer "B.Cu") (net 7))
 (segment (start 48.5 173.376915) (end 48.5 175.25) (width 0.5) (layer "F.Cu") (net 4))
 (segment (start 47.65 176.1) (end 46.418929 176.1) (width 0.5) (layer "F.Cu") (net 4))
 (segment (start 30.2 176.8) (end 35.041 171.959) (width 0.5) (layer "F.Cu") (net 4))
 (segment (start 35.041 171.959) (end 47.082085 171.959) (width 0.5) (layer "F.Cu") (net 4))
 (segment (start 47.082085 171.959) (end 48.5 173.376915) (width 0.5) (layer "F.Cu") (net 4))
 (segment (start 48.5 175.25) (end 47.65 176.1) (width 0.5) (layer "F.Cu") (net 4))
 (segment (start 67 103.75) (end 67.75 103) (width 0.5) (layer "B.Cu") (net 4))
 (segment (start 96.95 103) (end 97.45 103.5) (width 0.5) (layer "B.Cu") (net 4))
 (segment (start 67.75 103) (end 96.95 103) (width 0.5) (layer "B.Cu") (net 4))
 (segment (start 58.25 101.975) (end 60.025 103.75) (width 0.5) (layer "B.Cu") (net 4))
 (segment (start 60.025 103.75) (end 67 103.75) (width 0.5) (layer "B.Cu") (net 4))
 (segment (start 80.648214 180.76) (end 92.330357 180.76) (width 3) (layer "F.Cu") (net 14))
 (segment (start 80.648214 176.8) (end 92.330357 176.8) (width 3) (layer "F.Cu") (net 3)))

